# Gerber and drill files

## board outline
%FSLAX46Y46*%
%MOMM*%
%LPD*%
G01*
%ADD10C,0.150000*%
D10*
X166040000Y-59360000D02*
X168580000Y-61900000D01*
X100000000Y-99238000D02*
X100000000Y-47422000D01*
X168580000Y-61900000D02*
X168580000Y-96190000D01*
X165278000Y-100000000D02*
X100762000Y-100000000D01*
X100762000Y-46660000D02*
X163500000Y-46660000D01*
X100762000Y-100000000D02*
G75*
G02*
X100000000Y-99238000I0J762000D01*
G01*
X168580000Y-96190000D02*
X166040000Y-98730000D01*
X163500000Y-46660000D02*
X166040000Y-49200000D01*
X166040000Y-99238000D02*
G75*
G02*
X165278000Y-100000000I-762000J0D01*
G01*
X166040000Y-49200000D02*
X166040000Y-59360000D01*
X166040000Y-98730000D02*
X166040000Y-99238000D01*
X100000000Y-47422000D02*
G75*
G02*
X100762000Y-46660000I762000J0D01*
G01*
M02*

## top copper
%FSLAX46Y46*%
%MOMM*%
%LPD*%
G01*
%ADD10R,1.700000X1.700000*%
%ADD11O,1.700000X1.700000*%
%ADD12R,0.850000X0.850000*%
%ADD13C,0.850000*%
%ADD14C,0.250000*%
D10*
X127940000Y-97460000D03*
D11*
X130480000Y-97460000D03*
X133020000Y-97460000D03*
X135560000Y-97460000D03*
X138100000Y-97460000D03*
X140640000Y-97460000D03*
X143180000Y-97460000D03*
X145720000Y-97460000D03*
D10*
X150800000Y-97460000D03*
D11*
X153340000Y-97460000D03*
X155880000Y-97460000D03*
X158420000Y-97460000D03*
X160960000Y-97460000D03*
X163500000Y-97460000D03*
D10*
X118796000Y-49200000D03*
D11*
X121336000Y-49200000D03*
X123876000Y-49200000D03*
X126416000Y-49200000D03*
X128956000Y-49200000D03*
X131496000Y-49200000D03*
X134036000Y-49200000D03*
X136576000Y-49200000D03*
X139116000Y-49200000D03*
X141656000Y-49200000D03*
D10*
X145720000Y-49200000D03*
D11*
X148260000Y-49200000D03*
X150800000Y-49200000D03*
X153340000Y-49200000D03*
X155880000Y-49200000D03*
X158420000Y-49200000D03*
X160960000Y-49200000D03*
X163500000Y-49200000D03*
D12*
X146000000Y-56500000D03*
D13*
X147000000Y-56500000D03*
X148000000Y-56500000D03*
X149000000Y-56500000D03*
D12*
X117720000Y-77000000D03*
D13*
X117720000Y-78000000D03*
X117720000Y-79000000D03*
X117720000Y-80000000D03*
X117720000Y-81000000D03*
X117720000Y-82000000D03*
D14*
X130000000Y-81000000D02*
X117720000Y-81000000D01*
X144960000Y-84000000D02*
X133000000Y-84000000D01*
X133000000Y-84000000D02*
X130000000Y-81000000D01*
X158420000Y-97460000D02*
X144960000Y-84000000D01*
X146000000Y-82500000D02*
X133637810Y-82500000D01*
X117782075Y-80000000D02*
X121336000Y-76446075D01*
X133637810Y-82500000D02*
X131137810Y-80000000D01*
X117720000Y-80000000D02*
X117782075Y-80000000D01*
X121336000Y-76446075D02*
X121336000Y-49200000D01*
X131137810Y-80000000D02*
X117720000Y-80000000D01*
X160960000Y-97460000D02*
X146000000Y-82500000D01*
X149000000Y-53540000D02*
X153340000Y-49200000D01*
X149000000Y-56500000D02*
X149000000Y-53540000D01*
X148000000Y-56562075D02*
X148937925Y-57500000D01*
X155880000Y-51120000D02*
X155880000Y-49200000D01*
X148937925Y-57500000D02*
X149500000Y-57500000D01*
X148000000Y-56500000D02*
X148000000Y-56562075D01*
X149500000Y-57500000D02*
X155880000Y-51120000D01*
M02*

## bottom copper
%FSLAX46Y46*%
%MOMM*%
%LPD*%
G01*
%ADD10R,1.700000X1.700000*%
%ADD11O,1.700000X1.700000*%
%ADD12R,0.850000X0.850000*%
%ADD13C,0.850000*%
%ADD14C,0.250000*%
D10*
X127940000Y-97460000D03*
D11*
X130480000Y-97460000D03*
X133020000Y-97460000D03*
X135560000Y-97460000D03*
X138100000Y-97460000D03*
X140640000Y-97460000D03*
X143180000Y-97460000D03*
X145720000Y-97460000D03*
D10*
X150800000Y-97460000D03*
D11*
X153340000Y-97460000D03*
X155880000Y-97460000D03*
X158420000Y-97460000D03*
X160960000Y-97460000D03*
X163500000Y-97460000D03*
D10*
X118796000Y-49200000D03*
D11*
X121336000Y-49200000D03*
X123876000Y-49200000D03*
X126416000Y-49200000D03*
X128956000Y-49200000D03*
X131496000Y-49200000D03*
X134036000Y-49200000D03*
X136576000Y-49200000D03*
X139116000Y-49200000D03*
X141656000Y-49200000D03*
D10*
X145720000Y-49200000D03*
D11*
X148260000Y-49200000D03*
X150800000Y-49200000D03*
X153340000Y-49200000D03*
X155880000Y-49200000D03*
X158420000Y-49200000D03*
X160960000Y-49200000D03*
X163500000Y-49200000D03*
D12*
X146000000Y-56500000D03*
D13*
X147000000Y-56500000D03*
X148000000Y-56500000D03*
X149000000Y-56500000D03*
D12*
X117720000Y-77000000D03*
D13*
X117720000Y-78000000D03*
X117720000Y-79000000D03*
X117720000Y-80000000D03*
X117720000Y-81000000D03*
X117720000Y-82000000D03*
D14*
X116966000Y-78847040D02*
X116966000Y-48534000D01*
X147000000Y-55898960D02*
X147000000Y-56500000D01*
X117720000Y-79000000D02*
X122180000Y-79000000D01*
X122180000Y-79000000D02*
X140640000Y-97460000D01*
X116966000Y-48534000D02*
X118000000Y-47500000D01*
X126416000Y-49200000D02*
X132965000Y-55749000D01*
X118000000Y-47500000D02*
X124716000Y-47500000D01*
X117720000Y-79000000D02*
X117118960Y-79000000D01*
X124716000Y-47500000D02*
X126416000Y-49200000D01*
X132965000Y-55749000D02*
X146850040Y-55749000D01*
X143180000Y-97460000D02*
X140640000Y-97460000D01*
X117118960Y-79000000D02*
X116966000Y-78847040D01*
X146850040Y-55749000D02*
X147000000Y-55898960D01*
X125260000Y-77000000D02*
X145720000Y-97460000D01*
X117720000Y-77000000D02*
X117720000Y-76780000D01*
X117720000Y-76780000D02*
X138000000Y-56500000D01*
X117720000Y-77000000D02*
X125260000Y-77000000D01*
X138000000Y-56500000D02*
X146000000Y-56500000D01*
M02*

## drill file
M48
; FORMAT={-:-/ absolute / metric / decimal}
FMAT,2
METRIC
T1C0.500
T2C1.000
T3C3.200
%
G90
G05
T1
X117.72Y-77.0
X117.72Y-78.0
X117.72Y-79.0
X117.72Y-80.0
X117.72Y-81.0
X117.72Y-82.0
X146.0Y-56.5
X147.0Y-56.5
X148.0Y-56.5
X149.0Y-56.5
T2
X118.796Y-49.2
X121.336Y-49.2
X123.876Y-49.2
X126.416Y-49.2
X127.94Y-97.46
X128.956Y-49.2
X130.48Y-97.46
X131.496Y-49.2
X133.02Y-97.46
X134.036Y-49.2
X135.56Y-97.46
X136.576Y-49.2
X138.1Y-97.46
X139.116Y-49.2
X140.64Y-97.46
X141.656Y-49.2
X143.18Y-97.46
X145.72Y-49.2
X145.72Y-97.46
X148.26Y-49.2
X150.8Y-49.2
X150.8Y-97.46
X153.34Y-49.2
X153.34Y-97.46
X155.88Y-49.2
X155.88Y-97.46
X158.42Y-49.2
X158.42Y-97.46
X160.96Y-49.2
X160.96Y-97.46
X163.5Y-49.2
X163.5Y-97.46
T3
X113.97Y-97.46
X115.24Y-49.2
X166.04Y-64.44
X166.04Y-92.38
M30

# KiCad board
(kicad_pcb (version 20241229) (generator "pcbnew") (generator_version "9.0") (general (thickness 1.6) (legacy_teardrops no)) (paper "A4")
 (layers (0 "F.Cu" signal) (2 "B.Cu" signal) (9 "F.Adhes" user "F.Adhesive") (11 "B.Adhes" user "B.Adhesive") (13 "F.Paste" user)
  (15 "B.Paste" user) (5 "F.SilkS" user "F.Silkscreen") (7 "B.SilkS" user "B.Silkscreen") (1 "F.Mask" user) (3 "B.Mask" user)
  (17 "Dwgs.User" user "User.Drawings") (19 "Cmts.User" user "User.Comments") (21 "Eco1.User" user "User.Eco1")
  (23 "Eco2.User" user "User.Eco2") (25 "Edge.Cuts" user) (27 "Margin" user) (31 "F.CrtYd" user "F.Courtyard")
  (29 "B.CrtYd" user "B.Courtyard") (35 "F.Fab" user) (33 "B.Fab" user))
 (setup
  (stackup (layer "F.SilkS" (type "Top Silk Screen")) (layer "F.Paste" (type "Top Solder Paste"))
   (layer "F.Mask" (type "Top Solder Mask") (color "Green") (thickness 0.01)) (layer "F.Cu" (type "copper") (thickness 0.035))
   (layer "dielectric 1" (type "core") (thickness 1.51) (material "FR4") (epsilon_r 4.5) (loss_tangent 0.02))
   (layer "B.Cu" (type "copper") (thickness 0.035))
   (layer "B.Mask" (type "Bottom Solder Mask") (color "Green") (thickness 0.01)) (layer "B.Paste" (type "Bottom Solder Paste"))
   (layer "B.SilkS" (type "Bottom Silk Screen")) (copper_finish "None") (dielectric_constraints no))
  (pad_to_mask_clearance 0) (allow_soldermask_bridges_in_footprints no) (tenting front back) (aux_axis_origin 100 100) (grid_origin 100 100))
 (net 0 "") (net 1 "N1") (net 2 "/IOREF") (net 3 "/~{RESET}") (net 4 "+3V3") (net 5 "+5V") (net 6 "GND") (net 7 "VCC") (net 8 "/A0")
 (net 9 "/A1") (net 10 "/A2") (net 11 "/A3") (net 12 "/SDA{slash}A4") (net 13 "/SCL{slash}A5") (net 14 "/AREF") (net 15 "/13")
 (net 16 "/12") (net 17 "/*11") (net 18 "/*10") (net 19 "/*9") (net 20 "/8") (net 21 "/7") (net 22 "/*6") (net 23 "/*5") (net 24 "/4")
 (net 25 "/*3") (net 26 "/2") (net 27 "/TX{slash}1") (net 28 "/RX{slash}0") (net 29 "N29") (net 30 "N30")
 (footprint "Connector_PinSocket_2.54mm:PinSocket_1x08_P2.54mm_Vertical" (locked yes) (layer "F.Cu") (at 127.94 97.46 90)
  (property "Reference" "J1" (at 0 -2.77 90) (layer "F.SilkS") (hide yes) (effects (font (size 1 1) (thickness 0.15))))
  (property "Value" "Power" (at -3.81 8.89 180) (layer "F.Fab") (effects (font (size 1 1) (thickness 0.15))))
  (pad "1" thru_hole rect (at 0 0 90) (size 1.7 1.7) (drill 1) (layers "*.Cu" "*.Mask") (remove_unused_layers no) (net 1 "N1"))
  (pad "2" thru_hole oval (at 0 2.54 90) (size 1.7 1.7) (drill 1) (layers "*.Cu" "*.Mask") (remove_unused_layers no) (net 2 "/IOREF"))
  (pad "3" thru_hole oval (at 0 5.08 90) (size 1.7 1.7) (drill 1) (layers "*.Cu" "*.Mask") (remove_unused_layers no) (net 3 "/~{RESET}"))
  (pad "4" thru_hole oval (at 0 7.62 90) (size 1.7 1.7) (drill 1) (layers "*.Cu" "*.Mask") (remove_unused_layers no) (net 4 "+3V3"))
  (pad "5" thru_hole oval (at 0 10.16 90) (size 1.7 1.7) (drill 1) (layers "*.Cu" "*.Mask") (remove_unused_layers no) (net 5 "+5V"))
  (pad "6" thru_hole oval (at 0 12.7 90) (size 1.7 1.7) (drill 1) (layers "*.Cu" "*.Mask") (remove_unused_layers no) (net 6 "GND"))
  (pad "7" thru_hole oval (at 0 15.24 90) (size 1.7 1.7) (drill 1) (layers "*.Cu" "*.Mask") (remove_unused_layers no) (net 6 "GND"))
  (pad "8" thru_hole oval (at 0 17.78 90) (size 1.7 1.7) (drill 1) (layers "*.Cu" "*.Mask") (remove_unused_layers no) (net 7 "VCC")))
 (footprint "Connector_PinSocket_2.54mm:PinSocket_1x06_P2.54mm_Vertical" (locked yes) (layer "F.Cu") (at 150.8 97.46 90)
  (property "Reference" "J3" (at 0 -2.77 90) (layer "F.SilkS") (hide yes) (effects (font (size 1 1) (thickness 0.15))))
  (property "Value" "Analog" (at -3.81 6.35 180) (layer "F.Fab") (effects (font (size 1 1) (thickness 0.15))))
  (pad "1" thru_hole rect (at 0 0 90) (size 1.7 1.7) (drill 1) (layers "*.Cu" "*.Mask") (remove_unused_layers no) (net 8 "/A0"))
  (pad "2" thru_hole oval (at 0 2.54 90) (size 1.7 1.7) (drill 1) (layers "*.Cu" "*.Mask") (remove_unused_layers no) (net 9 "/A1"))
  (pad "3" thru_hole oval (at 0 5.08 90) (size 1.7 1.7) (drill 1) (layers "*.Cu" "*.Mask") (remove_unused_layers no) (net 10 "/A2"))
  (pad "4" thru_hole oval (at 0 7.62 90) (size 1.7 1.7) (drill 1) (layers "*.Cu" "*.Mask") (remove_unused_layers no) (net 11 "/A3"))
  (pad "5" thru_hole oval (at 0 10.16 90) (size 1.7 1.7) (drill 1) (layers "*.Cu" "*.Mask") (remove_unused_layers no)
   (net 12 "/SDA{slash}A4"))
  (pad "6" thru_hole oval (at 0 12.7 90) (size 1.7 1.7) (drill 1) (layers "*.Cu" "*.Mask") (remove_unused_layers no)
   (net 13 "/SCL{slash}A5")))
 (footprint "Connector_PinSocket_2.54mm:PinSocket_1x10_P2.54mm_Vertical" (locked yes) (layer "F.Cu") (at 118.796 49.2 90)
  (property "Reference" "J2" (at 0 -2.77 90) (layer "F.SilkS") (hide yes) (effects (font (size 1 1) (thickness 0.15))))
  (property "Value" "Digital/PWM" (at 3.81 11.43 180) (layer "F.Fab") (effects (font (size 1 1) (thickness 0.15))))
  (pad "1" thru_hole rect (at 0 0 90) (size 1.7 1.7) (drill 1) (layers "*.Cu" "*.Mask") (remove_unused_layers no) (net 13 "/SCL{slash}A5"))
  (pad "2" thru_hole oval (at 0 2.54 90) (size 1.7 1.7) (drill 1) (layers "*.Cu" "*.Mask") (remove_unused_layers no)
   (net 12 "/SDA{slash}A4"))
  (pad "3" thru_hole oval (at 0 5.08 90) (size 1.7 1.7) (drill 1) (layers "*.Cu" "*.Mask") (remove_unused_layers no) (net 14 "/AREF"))
  (pad "4" thru_hole oval (at 0 7.62 90) (size 1.7 1.7) (drill 1) (layers "*.Cu" "*.Mask") (remove_unused_layers no) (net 6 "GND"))
  (pad "5" thru_hole oval (at 0 10.16 90) (size 1.7 1.7) (drill 1) (layers "*.Cu" "*.Mask") (remove_unused_layers no) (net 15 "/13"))
  (pad "6" thru_hole oval (at 0 12.7 90) (size 1.7 1.7) (drill 1) (layers "*.Cu" "*.Mask") (remove_unused_layers no) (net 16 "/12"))
  (pad "7" thru_hole oval (at 0 15.24 90) (size 1.7 1.7) (drill 1) (layers "*.Cu" "*.Mask") (remove_unused_layers no) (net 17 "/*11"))
  (pad "8" thru_hole oval (at 0 17.78 90) (size 1.7 1.7) (drill 1) (layers "*.Cu" "*.Mask") (remove_unused_layers no) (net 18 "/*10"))
  (pad "9" thru_hole oval (at 0 20.32 90) (size 1.7 1.7) (drill 1) (layers "*.Cu" "*.Mask") (remove_unused_layers no) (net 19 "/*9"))
  (pad "10" thru_hole oval (at 0 22.86 90) (size 1.7 1.7) (drill 1) (layers "*.Cu" "*.Mask") (remove_unused_layers no) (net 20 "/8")))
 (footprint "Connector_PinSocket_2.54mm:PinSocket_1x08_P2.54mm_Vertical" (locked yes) (layer "F.Cu") (at 145.72 49.2 90)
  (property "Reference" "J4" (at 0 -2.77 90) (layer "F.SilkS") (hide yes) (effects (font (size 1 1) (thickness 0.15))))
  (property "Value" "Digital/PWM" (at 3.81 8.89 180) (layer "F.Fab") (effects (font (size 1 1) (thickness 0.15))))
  (pad "1" thru_hole rect (at 0 0 90) (size 1.7 1.7) (drill 1) (layers "*.Cu" "*.Mask") (remove_unused_layers no) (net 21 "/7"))
  (pad "2" thru_hole oval (at 0 2.54 90) (size 1.7 1.7) (drill 1) (layers "*.Cu" "*.Mask") (remove_unused_layers no) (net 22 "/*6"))
  (pad "3" thru_hole oval (at 0 5.08 90) (size 1.7 1.7) (drill 1) (layers "*.Cu" "*.Mask") (remove_unused_layers no) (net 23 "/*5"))
  (pad "4" thru_hole oval (at 0 7.62 90) (size 1.7 1.7) (drill 1) (layers "*.Cu" "*.Mask") (remove_unused_layers no) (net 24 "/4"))
  (pad "5" thru_hole oval (at 0 10.16 90) (size 1.7 1.7) (drill 1) (layers "*.Cu" "*.Mask") (remove_unused_layers no) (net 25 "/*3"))
  (pad "6" thru_hole oval (at 0 12.7 90) (size 1.7 1.7) (drill 1) (layers "*.Cu" "*.Mask") (remove_unused_layers no) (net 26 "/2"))
  (pad "7" thru_hole oval (at 0 15.24 90) (size 1.7 1.7) (drill 1) (layers "*.Cu" "*.Mask") (remove_unused_layers no) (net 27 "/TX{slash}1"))
  (pad "8" thru_hole oval (at 0 17.78 90) (size 1.7 1.7) (drill 1) (layers "*.Cu" "*.Mask") (remove_unused_layers no) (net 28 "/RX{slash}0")))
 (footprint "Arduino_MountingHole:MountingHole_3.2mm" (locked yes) (layer "F.Cu") (at 115.24 49.2)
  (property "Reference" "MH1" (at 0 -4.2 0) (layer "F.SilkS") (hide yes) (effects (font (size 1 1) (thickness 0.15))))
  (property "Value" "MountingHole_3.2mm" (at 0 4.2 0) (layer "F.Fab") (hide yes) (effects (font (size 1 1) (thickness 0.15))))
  (pad "" np_thru_hole circle (at 0 0) (size 3.2 3.2) (drill 3.2) (layers "*.Cu" "*.Mask")))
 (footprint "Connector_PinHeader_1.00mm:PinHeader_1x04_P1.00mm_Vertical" (layer "F.Cu") (at 146 56.5 90)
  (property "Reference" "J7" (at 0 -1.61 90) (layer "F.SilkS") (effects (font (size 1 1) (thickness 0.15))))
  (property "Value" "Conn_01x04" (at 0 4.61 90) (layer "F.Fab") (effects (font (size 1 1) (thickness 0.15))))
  (pad "1" thru_hole rect (at 0 0 90) (size 0.85 0.85) (drill 0.5) (layers "*.Cu" "*.Mask") (remove_unused_layers no) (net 7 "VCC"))
  (pad "2" thru_hole circle (at 0 1 90) (size 0.85 0.85) (drill 0.5) (layers "*.Cu" "*.Mask") (remove_unused_layers no) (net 6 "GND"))
  (pad "3" thru_hole circle (at 0 2 90) (size 0.85 0.85) (drill 0.5) (layers "*.Cu" "*.Mask") (remove_unused_layers no) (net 25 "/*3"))
  (pad "4" thru_hole circle (at 0 3 90) (size 0.85 0.85) (drill 0.5) (layers "*.Cu" "*.Mask") (remove_unused_layers no) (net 24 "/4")))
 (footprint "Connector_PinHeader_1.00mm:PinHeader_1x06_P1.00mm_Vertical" (layer "F.Cu") (at 117.72 77)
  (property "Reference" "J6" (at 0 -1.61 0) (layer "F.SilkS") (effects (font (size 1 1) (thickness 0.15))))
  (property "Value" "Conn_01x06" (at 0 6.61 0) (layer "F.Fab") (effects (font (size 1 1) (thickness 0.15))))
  (pad "1" thru_hole rect (at 0 0) (size 0.85 0.85) (drill 0.5) (layers "*.Cu" "*.Mask") (remove_unused_layers no) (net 7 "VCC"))
  (pad "2" thru_hole circle (at 0 1) (size 0.85 0.85) (drill 0.5) (layers "*.Cu" "*.Mask") (remove_unused_layers no) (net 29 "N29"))
  (pad "3" thru_hole circle (at 0 2) (size 0.85 0.85) (drill 0.5) (layers "*.Cu" "*.Mask") (remove_unused_layers no) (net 6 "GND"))
  (pad "4" thru_hole circle (at 0 3) (size 0.85 0.85) (drill 0.5) (layers "*.Cu" "*.Mask") (remove_unused_layers no)
   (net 12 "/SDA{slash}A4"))
  (pad "5" thru_hole circle (at 0 4) (size 0.85 0.85) (drill 0.5) (layers "*.Cu" "*.Mask") (remove_unused_layers no) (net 11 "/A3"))
  (pad "6" thru_hole circle (at 0 5) (size 0.85 0.85) (drill 0.5) (layers "*.Cu" "*.Mask") (remove_unused_layers no) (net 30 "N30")))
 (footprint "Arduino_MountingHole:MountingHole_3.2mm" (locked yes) (layer "F.Cu") (at 113.97 97.46)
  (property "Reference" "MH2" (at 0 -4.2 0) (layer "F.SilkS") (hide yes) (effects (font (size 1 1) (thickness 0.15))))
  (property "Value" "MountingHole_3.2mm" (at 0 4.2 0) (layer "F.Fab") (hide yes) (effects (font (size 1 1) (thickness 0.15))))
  (pad "" np_thru_hole circle (at 0 0) (size 3.2 3.2) (drill 3.2) (layers "*.Cu" "*.Mask")))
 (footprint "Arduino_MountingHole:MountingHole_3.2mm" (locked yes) (layer "F.Cu") (at 166.04 64.44)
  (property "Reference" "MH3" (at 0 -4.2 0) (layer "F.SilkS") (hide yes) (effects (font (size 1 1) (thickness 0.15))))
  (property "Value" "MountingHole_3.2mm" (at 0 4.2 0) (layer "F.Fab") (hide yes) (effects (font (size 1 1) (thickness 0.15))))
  (pad "" np_thru_hole circle (at 0 0) (size 3.2 3.2) (drill 3.2) (layers "*.Cu" "*.Mask")))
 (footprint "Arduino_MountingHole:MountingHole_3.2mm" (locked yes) (layer "F.Cu") (at 166.04 92.38)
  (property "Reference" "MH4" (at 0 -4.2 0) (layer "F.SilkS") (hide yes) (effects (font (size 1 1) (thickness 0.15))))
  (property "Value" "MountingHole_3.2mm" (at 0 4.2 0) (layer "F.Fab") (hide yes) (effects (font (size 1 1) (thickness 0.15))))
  (pad "" np_thru_hole circle (at 0 0) (size 3.2 3.2) (drill 3.2) (layers "*.Cu" "*.Mask")))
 (gr_line (start 166.04 59.36) (end 168.58 61.9) (stroke (width 0.15) (type solid)) (layer "Edge.Cuts"))
 (gr_line (start 100 99.238) (end 100 47.422) (stroke (width 0.15) (type solid)) (layer "Edge.Cuts"))
 (gr_line (start 168.58 61.9) (end 168.58 96.19) (stroke (width 0.15) (type solid)) (layer "Edge.Cuts"))
 (gr_line (start 165.278 100) (end 100.762 100) (stroke (width 0.15) (type solid)) (layer "Edge.Cuts"))
 (gr_line (start 100.762 46.66) (end 163.5 46.66) (stroke (width 0.15) (type solid)) (layer "Edge.Cuts"))
 (gr_arc (start 100.762 100) (mid 100.223185 99.776815) (end 100 99.238) (stroke (width 0.15) (type solid)) (layer "Edge.Cuts"))
 (gr_line (start 168.58 96.19) (end 166.04 98.73) (stroke (width 0.15) (type solid)) (layer "Edge.Cuts"))
 (gr_line (start 163.5 46.66) (end 166.04 49.2) (stroke (width 0.15) (type solid)) (layer "Edge.Cuts"))
 (gr_arc (start 166.04 99.238) (mid 165.816815 99.776815) (end 165.278 100) (stroke (width 0.15) (type solid)) (layer "Edge.Cuts"))
 (gr_line (start 166.04 49.2) (end 166.04 59.36) (stroke (width 0.15) (type solid)) (layer "Edge.Cuts"))
 (gr_line (start 166.04 98.73) (end 166.04 99.238) (stroke (width 0.15) (type solid)) (layer "Edge.Cuts"))
 (gr_arc (start 100 47.422) (mid 100.223185 46.883185) (end 100.762 46.66) (stroke (width 0.15) (type solid)) (layer "Edge.Cuts"))
 (segment (start 116.966 78.84704) (end 116.966 48.534) (width 0.25) (layer "B.Cu") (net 6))
 (segment (start 147 55.89896) (end 147 56.5) (width 0.25) (layer "B.Cu") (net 6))
 (segment (start 117.72 79) (end 122.18 79) (width 0.25) (layer "B.Cu") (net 6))
 (segment (start 122.18 79) (end 140.64 97.46) (width 0.25) (layer "B.Cu") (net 6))
 (segment (start 116.966 48.534) (end 118 47.5) (width 0.25) (layer "B.Cu") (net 6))
 (segment (start 126.416 49.2) (end 132.965 55.749) (width 0.25) (layer "B.Cu") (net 6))
 (segment (start 118 47.5) (end 124.716 47.5) (width 0.25) (layer "B.Cu") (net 6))
 (segment (start 117.72 79) (end 117.11896 79) (width 0.25) (layer "B.Cu") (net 6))
 (segment (start 124.716 47.5) (end 126.416 49.2) (width 0.25) (layer "B.Cu") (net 6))
 (segment (start 132.965 55.749) (end 146.85004 55.749) (width 0.25) (layer "B.Cu") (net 6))
 (segment (start 143.18 97.46) (end 140.64 97.46) (width 0.25) (layer "B.Cu") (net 6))
 (segment (start 117.11896 79) (end 116.966 78.84704) (width 0.25) (layer "B.Cu") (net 6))
 (segment (start 146.85004 55.749) (end 147 55.89896) (width 0.25) (layer "B.Cu") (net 6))
 (segment (start 130 81) (end 117.72 81) (width 0.25) (layer "F.Cu") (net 11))
 (segment (start 144.96 84) (end 133 84) (width 0.25) (layer "F.Cu") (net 11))
 (segment (start 133 84) (end 130 81) (width 0.25) (layer "F.Cu") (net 11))
 (segment (start 158.42 97.46) (end 144.96 84) (width 0.25) (layer "F.Cu") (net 11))
 (segment (start 146 82.5) (end 133.63781 82.5) (width 0.25) (layer "F.Cu") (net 12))
 (segment (start 117.782075 80) (end 121.336 76.446075) (width 0.25) (layer "F.Cu") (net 12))
 (segment (start 133.63781 82.5) (end 131.13781 80) (width 0.25) (layer "F.Cu") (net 12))
 (segment (start 117.72 80) (end 117.782075 80) (width 0.25) (layer "F.Cu") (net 12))
 (segment (start 121.336 76.446075) (end 121.336 49.2) (width 0.25) (layer "F.Cu") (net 12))
 (segment (start 131.13781 80) (end 117.72 80) (width 0.25) (layer "F.Cu") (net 12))
 (segment (start 160.96 97.46) (end 146 82.5) (width 0.25) (layer "F.Cu") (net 12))
 (segment (start 149 53.54) (end 153.34 49.2) (width 0.25) (layer "F.Cu") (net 24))
 (segment (start 149 56.5) (end 149 53.54) (width 0.25) (layer "F.Cu") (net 24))
 (segment (start 148 56.562075) (end 148.937925 57.5) (width 0.25) (layer "F.Cu") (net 25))
 (segment (start 155.88 51.12) (end 155.88 49.2) (width 0.25) (layer "F.Cu") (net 25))
 (segment (start 148.937925 57.5) (end 149.5 57.5) (width 0.25) (layer "F.Cu") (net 25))
 (segment (start 148 56.5) (end 148 56.562075) (width 0.25) (layer "F.Cu") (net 25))
 (segment (start 149.5 57.5) (end 155.88 51.12) (width 0.25) (layer "F.Cu") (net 25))
 (segment (start 125.26 77) (end 145.72 97.46) (width 0.25) (layer "B.Cu") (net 7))
 (segment (start 117.72 77) (end 117.72 76.78) (width 0.25) (layer "B.Cu") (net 7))
 (segment (start 117.72 76.78) (end 138 56.5) (width 0.25) (layer "B.Cu") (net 7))
 (segment (start 117.72 77) (end 125.26 77) (width 0.25) (layer "B.Cu") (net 7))
 (segment (start 138 56.5) (end 146 56.5) (width 0.25) (layer "B.Cu") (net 7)))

